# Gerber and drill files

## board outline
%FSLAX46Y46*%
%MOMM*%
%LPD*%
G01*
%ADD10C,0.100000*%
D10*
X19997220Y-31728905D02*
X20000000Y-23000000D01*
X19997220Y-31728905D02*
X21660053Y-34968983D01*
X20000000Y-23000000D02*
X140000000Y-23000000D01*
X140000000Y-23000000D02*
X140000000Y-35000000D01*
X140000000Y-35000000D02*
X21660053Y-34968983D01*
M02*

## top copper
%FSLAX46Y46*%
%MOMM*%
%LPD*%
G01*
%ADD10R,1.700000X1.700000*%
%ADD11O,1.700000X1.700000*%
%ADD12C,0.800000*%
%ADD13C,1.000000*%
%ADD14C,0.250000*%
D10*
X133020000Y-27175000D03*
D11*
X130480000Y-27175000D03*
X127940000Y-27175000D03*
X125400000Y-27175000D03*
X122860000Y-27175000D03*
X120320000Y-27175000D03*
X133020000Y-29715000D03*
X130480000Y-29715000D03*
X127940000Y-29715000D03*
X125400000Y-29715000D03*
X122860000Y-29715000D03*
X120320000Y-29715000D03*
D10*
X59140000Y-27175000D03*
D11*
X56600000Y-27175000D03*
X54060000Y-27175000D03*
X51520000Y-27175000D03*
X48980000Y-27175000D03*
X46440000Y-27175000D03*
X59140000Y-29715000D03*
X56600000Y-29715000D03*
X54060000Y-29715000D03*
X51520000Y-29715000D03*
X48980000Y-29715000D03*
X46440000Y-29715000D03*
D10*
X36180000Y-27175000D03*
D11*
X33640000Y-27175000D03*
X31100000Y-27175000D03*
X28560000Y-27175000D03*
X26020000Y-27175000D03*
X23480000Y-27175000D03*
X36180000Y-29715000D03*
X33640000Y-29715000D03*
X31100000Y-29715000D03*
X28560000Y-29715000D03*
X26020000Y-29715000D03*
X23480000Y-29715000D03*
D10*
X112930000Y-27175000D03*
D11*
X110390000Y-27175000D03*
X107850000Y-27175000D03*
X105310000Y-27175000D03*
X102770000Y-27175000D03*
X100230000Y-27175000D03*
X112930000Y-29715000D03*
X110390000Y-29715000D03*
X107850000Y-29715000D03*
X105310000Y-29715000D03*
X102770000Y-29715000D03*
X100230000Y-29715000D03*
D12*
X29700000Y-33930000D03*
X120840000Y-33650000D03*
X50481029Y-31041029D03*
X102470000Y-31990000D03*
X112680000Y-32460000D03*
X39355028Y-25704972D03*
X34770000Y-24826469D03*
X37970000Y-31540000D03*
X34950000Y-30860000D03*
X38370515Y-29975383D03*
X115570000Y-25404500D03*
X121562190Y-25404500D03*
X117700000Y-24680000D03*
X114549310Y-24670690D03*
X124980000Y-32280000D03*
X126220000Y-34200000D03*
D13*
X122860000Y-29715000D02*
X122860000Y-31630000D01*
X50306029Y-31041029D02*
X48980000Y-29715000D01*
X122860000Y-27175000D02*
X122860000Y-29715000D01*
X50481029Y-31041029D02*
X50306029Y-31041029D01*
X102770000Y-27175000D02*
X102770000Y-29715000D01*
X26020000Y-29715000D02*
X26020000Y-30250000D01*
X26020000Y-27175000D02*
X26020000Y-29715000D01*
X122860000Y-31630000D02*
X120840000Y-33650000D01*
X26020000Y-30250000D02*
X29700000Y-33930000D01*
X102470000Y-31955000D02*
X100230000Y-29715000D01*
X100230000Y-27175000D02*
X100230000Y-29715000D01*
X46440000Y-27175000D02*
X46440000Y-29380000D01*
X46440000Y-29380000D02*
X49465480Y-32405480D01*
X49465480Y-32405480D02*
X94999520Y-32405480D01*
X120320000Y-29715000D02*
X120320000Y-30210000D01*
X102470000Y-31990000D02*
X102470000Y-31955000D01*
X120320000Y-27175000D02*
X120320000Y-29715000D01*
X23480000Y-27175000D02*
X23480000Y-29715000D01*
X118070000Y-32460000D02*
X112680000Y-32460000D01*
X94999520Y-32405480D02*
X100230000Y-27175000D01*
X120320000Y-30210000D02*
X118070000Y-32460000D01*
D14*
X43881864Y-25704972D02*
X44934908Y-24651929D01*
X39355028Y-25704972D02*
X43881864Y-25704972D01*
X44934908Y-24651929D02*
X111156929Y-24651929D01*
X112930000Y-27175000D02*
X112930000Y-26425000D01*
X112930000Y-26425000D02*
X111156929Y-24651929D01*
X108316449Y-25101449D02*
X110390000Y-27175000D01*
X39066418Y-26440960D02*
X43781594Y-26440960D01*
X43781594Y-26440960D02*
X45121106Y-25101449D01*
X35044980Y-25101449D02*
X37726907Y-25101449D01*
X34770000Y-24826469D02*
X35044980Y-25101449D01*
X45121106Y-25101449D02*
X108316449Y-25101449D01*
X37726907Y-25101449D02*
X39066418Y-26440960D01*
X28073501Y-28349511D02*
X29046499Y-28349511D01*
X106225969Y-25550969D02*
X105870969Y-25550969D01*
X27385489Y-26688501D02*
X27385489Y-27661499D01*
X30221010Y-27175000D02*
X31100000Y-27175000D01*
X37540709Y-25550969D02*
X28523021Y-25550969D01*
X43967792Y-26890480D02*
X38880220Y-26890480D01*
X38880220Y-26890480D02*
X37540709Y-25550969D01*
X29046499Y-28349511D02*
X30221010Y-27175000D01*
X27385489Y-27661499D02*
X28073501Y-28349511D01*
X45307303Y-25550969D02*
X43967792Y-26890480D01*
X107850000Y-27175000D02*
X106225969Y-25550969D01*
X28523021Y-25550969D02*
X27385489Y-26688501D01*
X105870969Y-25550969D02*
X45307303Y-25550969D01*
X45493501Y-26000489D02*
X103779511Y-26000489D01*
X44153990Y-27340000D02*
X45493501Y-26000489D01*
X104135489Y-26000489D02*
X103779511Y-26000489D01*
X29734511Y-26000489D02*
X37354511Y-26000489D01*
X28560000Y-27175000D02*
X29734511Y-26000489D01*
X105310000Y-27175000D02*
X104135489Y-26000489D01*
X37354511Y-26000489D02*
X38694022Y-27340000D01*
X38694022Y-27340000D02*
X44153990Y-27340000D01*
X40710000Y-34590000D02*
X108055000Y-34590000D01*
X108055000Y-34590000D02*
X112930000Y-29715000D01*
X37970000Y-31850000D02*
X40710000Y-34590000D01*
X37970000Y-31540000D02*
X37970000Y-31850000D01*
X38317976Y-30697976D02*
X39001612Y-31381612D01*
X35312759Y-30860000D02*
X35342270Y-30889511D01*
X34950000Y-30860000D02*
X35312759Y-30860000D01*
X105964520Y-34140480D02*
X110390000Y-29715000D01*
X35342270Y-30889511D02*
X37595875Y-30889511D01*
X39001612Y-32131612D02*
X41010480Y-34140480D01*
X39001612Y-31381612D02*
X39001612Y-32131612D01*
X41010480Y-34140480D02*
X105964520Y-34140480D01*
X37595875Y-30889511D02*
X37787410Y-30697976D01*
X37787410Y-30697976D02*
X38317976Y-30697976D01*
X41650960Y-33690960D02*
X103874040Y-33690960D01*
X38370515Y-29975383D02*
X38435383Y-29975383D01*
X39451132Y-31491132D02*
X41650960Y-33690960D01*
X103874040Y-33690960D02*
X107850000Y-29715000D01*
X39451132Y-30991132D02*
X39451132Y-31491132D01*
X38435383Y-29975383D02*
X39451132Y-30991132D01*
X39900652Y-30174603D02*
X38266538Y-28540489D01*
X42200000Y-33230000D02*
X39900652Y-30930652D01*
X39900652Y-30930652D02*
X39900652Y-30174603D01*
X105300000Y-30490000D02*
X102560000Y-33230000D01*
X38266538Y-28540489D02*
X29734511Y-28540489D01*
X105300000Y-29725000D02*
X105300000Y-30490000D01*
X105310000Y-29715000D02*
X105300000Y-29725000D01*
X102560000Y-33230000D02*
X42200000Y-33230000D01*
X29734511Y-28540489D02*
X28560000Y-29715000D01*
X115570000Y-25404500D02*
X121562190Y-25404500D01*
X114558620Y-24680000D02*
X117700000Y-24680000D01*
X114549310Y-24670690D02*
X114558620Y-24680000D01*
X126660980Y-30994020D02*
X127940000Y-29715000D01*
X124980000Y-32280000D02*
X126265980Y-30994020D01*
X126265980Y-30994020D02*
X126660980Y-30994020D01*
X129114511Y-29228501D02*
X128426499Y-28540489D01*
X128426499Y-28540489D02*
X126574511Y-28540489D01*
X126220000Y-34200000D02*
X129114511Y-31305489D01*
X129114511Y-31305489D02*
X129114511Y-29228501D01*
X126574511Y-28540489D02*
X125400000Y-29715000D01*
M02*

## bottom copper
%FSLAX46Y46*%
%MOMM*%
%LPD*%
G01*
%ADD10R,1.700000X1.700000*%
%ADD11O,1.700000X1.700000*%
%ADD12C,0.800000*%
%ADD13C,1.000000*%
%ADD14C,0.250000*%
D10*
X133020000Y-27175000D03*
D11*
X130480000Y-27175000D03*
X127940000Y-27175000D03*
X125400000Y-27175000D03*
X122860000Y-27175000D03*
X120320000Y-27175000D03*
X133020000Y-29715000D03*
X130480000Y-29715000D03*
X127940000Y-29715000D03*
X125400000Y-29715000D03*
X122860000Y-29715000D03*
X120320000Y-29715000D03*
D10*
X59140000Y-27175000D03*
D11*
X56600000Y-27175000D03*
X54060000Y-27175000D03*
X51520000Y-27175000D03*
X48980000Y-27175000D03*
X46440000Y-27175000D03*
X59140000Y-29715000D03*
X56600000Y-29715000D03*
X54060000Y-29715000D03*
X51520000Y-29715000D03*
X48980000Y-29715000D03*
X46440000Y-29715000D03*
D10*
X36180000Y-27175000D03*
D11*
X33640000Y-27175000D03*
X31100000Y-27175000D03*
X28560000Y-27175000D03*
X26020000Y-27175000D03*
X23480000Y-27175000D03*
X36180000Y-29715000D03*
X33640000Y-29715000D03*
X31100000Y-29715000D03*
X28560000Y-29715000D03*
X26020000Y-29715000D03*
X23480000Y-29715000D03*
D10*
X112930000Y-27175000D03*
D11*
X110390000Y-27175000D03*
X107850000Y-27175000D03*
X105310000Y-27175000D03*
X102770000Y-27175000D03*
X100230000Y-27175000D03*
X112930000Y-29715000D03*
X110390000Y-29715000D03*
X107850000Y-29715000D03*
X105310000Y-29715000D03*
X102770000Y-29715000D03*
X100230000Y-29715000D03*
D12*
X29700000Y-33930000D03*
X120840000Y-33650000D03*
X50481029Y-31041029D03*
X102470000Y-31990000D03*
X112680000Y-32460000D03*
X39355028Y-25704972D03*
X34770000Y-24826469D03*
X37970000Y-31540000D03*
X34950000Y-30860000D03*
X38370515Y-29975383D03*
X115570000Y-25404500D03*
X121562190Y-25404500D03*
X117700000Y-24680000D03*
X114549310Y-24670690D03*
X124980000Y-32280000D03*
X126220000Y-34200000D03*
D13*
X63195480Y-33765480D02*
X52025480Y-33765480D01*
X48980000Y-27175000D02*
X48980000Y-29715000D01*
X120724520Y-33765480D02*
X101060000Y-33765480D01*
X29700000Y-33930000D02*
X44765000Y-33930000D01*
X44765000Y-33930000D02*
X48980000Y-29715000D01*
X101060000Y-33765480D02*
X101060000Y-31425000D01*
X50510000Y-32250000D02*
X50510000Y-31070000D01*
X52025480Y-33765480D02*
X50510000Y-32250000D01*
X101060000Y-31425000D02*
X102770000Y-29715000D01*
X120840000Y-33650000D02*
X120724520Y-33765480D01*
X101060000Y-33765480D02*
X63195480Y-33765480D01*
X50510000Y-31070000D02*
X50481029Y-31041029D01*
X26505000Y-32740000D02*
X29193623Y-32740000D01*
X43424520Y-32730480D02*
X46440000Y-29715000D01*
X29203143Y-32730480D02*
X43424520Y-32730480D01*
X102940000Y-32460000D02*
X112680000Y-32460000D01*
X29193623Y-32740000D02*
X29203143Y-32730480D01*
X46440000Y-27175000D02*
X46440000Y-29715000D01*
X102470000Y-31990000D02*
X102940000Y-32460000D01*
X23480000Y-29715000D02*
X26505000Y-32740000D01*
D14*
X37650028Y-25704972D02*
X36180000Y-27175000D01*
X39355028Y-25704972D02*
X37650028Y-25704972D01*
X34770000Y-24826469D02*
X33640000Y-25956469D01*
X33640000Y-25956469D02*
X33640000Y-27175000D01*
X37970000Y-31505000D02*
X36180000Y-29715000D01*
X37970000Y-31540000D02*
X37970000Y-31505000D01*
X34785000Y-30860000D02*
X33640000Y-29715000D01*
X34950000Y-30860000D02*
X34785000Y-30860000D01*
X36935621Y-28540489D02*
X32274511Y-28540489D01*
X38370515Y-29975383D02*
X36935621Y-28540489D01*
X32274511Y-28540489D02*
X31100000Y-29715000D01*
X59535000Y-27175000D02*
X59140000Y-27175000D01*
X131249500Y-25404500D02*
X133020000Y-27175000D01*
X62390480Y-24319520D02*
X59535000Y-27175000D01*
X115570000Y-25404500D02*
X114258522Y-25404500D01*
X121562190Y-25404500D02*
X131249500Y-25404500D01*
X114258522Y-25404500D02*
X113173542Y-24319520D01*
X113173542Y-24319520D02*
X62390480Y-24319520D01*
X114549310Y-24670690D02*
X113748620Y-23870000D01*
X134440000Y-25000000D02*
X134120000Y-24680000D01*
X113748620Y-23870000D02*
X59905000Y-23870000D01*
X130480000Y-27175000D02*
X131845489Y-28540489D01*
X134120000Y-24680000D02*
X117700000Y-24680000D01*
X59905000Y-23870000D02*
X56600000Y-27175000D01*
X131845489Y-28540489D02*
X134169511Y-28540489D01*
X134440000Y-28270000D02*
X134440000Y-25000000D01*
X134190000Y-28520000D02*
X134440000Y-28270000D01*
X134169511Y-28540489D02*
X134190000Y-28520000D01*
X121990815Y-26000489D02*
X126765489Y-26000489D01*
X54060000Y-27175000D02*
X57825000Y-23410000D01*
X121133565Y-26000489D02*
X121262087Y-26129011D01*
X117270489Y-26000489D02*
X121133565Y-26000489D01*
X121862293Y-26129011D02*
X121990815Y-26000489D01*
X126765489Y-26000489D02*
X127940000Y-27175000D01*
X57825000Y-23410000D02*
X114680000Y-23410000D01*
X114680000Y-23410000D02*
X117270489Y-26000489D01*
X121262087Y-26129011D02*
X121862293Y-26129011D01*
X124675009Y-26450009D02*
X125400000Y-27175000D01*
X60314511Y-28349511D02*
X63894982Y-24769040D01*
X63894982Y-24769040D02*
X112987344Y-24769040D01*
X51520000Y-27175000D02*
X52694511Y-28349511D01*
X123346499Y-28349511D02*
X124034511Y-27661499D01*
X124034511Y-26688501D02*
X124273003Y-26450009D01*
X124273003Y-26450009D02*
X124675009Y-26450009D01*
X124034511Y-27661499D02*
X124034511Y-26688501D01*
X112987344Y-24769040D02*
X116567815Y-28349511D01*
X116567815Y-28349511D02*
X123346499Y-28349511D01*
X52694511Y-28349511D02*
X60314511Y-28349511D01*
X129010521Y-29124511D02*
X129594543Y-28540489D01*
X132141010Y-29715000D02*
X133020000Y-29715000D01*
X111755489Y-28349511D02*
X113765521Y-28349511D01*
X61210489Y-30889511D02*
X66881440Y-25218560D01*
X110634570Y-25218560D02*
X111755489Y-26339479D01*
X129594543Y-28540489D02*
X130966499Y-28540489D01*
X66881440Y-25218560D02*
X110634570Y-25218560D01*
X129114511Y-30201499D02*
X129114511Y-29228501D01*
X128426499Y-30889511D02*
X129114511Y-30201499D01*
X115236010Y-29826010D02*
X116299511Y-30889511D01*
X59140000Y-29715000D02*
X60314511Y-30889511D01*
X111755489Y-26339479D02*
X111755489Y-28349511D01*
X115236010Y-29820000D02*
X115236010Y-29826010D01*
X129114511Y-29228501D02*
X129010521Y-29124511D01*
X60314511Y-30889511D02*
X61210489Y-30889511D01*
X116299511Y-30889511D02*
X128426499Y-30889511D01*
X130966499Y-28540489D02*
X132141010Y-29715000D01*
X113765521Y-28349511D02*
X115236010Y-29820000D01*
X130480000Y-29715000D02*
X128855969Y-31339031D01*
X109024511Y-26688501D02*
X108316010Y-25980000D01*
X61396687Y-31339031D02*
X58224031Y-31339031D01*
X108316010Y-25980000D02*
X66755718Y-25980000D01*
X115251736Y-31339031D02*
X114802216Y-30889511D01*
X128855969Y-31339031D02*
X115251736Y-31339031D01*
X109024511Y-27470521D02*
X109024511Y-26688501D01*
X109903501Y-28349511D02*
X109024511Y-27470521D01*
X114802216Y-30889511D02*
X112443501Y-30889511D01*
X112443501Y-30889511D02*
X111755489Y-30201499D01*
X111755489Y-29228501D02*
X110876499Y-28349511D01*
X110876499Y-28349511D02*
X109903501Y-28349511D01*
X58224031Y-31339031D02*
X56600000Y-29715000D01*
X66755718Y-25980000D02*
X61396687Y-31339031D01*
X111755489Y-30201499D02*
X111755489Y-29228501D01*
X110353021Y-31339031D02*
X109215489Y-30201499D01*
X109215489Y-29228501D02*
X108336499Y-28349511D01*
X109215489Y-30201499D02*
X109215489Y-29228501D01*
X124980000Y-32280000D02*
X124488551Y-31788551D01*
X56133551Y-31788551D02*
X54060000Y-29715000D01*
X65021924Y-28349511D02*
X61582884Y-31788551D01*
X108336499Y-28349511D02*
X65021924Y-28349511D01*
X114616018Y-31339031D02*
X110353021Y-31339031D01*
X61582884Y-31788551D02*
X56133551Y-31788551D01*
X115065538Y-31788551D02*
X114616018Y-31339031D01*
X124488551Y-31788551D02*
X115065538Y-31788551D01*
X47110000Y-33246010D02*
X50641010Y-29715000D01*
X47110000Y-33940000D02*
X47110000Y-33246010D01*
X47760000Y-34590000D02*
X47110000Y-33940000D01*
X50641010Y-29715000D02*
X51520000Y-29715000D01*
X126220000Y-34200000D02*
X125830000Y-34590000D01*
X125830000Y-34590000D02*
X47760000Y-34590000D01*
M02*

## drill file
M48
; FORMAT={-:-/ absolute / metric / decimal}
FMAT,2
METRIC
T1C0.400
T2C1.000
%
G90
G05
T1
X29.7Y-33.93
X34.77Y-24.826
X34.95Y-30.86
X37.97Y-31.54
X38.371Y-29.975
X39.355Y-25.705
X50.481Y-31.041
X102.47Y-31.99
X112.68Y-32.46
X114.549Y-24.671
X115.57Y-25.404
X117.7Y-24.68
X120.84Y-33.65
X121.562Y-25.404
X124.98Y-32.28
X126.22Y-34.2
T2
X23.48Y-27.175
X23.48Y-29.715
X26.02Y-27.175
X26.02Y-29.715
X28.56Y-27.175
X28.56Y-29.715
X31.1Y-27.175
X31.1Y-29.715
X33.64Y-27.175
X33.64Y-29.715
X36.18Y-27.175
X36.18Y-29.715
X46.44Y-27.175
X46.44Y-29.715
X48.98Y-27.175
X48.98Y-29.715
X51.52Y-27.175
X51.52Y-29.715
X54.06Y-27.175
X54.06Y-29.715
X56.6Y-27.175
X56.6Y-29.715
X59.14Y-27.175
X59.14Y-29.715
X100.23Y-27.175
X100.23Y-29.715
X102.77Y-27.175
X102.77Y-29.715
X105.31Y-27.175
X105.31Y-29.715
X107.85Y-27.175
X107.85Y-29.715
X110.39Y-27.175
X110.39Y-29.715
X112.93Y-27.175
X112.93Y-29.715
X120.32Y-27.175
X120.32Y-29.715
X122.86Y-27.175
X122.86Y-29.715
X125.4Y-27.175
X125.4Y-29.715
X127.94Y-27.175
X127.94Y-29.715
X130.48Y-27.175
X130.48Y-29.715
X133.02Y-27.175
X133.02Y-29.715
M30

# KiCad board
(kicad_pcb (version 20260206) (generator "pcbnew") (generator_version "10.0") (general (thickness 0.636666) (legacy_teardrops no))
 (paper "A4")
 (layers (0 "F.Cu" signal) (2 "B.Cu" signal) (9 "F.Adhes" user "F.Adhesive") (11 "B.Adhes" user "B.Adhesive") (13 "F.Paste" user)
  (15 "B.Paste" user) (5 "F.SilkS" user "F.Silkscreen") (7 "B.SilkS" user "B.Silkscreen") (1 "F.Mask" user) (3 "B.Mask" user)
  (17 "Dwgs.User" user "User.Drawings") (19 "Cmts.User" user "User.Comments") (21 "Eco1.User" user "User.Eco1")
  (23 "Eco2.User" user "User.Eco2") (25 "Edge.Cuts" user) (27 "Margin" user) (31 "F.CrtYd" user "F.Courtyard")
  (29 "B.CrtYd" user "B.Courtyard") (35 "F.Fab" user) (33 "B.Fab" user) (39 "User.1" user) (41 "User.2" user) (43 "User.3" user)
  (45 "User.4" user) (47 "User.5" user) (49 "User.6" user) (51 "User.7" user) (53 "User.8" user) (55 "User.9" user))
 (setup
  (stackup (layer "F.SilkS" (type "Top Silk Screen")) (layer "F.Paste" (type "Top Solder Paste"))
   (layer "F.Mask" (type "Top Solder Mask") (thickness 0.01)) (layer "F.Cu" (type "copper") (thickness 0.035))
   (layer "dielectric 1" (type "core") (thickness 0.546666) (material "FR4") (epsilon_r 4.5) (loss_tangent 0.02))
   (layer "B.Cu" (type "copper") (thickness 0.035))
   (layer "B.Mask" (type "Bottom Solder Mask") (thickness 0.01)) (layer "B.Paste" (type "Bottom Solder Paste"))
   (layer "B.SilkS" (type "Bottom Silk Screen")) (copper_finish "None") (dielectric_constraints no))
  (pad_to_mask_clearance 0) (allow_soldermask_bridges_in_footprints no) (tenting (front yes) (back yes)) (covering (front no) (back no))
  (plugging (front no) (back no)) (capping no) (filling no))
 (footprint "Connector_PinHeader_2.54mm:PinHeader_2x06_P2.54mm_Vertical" (layer "F.Cu") (at 133.02 27.175 -90)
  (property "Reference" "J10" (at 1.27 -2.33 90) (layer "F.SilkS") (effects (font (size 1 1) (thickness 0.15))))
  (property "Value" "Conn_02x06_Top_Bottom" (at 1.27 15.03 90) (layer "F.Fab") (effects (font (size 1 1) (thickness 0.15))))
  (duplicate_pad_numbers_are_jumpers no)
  (pad "1" thru_hole rect (at 0 0 270) (size 1.7 1.7) (drill 1) (layers "*.Cu" "*.Mask") (remove_unused_layers no) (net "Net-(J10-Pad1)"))
  (pad "2" thru_hole oval (at 0 2.54 270) (size 1.7 1.7) (drill 1) (layers "*.Cu" "*.Mask") (remove_unused_layers no) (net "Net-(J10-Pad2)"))
  (pad "3" thru_hole oval (at 0 5.08 270) (size 1.7 1.7) (drill 1) (layers "*.Cu" "*.Mask") (remove_unused_layers no) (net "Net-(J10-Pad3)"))
  (pad "4" thru_hole oval (at 0 7.62 270) (size 1.7 1.7) (drill 1) (layers "*.Cu" "*.Mask") (remove_unused_layers no) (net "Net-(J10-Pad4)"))
  (pad "5" thru_hole oval (at 0 10.16 270) (size 1.7 1.7) (drill 1) (layers "*.Cu" "*.Mask") (remove_unused_layers no) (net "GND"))
  (pad "6" thru_hole oval (at 0 12.7 270) (size 1.7 1.7) (drill 1) (layers "*.Cu" "*.Mask") (remove_unused_layers no) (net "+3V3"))
  (pad "7" thru_hole oval (at 2.54 0 270) (size 1.7 1.7) (drill 1) (layers "*.Cu" "*.Mask") (remove_unused_layers no) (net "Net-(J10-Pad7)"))
  (pad "8" thru_hole oval (at 2.54 2.54 270) (size 1.7 1.7) (drill 1) (layers "*.Cu" "*.Mask") (remove_unused_layers no)
   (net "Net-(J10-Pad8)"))
  (pad "9" thru_hole oval (at 2.54 5.08 270) (size 1.7 1.7) (drill 1) (layers "*.Cu" "*.Mask") (remove_unused_layers no)
   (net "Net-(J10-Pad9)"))
  (pad "10" thru_hole oval (at 2.54 7.62 270) (size 1.7 1.7) (drill 1) (layers "*.Cu" "*.Mask") (remove_unused_layers no)
   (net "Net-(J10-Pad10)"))
  (pad "11" thru_hole oval (at 2.54 10.16 270) (size 1.7 1.7) (drill 1) (layers "*.Cu" "*.Mask") (remove_unused_layers no) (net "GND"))
  (pad "12" thru_hole oval (at 2.54 12.7 270) (size 1.7 1.7) (drill 1) (layers "*.Cu" "*.Mask") (remove_unused_layers no) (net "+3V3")))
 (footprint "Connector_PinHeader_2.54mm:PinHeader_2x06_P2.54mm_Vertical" (layer "F.Cu") (at 59.14 27.175 -90)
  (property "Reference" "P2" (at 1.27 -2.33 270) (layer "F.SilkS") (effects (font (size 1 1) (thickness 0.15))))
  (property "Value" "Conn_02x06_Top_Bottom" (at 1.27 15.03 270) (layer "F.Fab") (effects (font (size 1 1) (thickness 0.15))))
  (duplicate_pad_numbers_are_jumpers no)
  (pad "1" thru_hole rect (at 0 0 270) (size 1.7 1.7) (drill 1) (layers "*.Cu" "*.Mask") (remove_unused_layers no) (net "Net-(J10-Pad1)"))
  (pad "2" thru_hole oval (at 0 2.54 270) (size 1.7 1.7) (drill 1) (layers "*.Cu" "*.Mask") (remove_unused_layers no) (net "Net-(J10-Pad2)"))
  (pad "3" thru_hole oval (at 0 5.08 270) (size 1.7 1.7) (drill 1) (layers "*.Cu" "*.Mask") (remove_unused_layers no) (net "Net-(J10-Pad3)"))
  (pad "4" thru_hole oval (at 0 7.62 270) (size 1.7 1.7) (drill 1) (layers "*.Cu" "*.Mask") (remove_unused_layers no) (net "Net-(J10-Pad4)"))
  (pad "5" thru_hole oval (at 0 10.16 270) (size 1.7 1.7) (drill 1) (layers "*.Cu" "*.Mask") (remove_unused_layers no) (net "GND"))
  (pad "6" thru_hole oval (at 0 12.7 270) (size 1.7 1.7) (drill 1) (layers "*.Cu" "*.Mask") (remove_unused_layers no) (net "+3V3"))
  (pad "7" thru_hole oval (at 2.54 0 270) (size 1.7 1.7) (drill 1) (layers "*.Cu" "*.Mask") (remove_unused_layers no) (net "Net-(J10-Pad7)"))
  (pad "8" thru_hole oval (at 2.54 2.54 270) (size 1.7 1.7) (drill 1) (layers "*.Cu" "*.Mask") (remove_unused_layers no)
   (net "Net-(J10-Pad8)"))
  (pad "9" thru_hole oval (at 2.54 5.08 270) (size 1.7 1.7) (drill 1) (layers "*.Cu" "*.Mask") (remove_unused_layers no)
   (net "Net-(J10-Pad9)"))
  (pad "10" thru_hole oval (at 2.54 7.62 270) (size 1.7 1.7) (drill 1) (layers "*.Cu" "*.Mask") (remove_unused_layers no)
   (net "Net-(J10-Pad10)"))
  (pad "11" thru_hole oval (at 2.54 10.16 270) (size 1.7 1.7) (drill 1) (layers "*.Cu" "*.Mask") (remove_unused_layers no) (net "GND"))
  (pad "12" thru_hole oval (at 2.54 12.7 270) (size 1.7 1.7) (drill 1) (layers "*.Cu" "*.Mask") (remove_unused_layers no) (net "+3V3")))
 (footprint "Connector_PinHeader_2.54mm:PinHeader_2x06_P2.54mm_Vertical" (layer "F.Cu") (at 36.18 27.175 -90)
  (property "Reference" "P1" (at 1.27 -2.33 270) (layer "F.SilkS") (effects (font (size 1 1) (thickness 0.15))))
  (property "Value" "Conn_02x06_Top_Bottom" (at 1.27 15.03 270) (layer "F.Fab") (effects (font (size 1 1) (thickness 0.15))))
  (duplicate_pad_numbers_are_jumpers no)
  (pad "1" thru_hole rect (at 0 0 270) (size 1.7 1.7) (drill 1) (layers "*.Cu" "*.Mask") (remove_unused_layers no) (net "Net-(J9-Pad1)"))
  (pad "2" thru_hole oval (at 0 2.54 270) (size 1.7 1.7) (drill 1) (layers "*.Cu" "*.Mask") (remove_unused_layers no) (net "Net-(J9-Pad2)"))
  (pad "3" thru_hole oval (at 0 5.08 270) (size 1.7 1.7) (drill 1) (layers "*.Cu" "*.Mask") (remove_unused_layers no) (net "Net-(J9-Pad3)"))
  (pad "4" thru_hole oval (at 0 7.62 270) (size 1.7 1.7) (drill 1) (layers "*.Cu" "*.Mask") (remove_unused_layers no) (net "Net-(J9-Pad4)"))
  (pad "5" thru_hole oval (at 0 10.16 270) (size 1.7 1.7) (drill 1) (layers "*.Cu" "*.Mask") (remove_unused_layers no) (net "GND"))
  (pad "6" thru_hole oval (at 0 12.7 270) (size 1.7 1.7) (drill 1) (layers "*.Cu" "*.Mask") (remove_unused_layers no) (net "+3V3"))
  (pad "7" thru_hole oval (at 2.54 0 270) (size 1.7 1.7) (drill 1) (layers "*.Cu" "*.Mask") (remove_unused_layers no) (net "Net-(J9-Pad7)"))
  (pad "8" thru_hole oval (at 2.54 2.54 270) (size 1.7 1.7) (drill 1) (layers "*.Cu" "*.Mask") (remove_unused_layers no)
   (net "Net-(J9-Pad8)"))
  (pad "9" thru_hole oval (at 2.54 5.08 270) (size 1.7 1.7) (drill 1) (layers "*.Cu" "*.Mask") (remove_unused_layers no)
   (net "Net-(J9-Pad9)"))
  (pad "10" thru_hole oval (at 2.54 7.62 270) (size 1.7 1.7) (drill 1) (layers "*.Cu" "*.Mask") (remove_unused_layers no)
   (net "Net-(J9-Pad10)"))
  (pad "11" thru_hole oval (at 2.54 10.16 270) (size 1.7 1.7) (drill 1) (layers "*.Cu" "*.Mask") (remove_unused_layers no) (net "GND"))
  (pad "12" thru_hole oval (at 2.54 12.7 270) (size 1.7 1.7) (drill 1) (layers "*.Cu" "*.Mask") (remove_unused_layers no) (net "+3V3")))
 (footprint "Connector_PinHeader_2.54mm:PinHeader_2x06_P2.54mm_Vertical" (layer "F.Cu") (at 112.93 27.175 -90)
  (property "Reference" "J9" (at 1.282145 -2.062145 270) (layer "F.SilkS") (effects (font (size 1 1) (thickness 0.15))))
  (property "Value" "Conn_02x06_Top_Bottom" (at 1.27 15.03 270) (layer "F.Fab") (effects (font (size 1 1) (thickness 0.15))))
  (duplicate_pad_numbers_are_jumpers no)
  (pad "1" thru_hole rect (at 0 0 270) (size 1.7 1.7) (drill 1) (layers "*.Cu" "*.Mask") (remove_unused_layers no) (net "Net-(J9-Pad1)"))
  (pad "2" thru_hole oval (at 0 2.54 270) (size 1.7 1.7) (drill 1) (layers "*.Cu" "*.Mask") (remove_unused_layers no) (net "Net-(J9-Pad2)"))
  (pad "3" thru_hole oval (at 0 5.08 270) (size 1.7 1.7) (drill 1) (layers "*.Cu" "*.Mask") (remove_unused_layers no) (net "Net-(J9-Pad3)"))
  (pad "4" thru_hole oval (at 0 7.62 270) (size 1.7 1.7) (drill 1) (layers "*.Cu" "*.Mask") (remove_unused_layers no) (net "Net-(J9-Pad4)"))
  (pad "5" thru_hole oval (at 0 10.16 270) (size 1.7 1.7) (drill 1) (layers "*.Cu" "*.Mask") (remove_unused_layers no) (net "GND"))
  (pad "6" thru_hole oval (at 0 12.7 270) (size 1.7 1.7) (drill 1) (layers "*.Cu" "*.Mask") (remove_unused_layers no) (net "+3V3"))
  (pad "7" thru_hole oval (at 2.54 0 270) (size 1.7 1.7) (drill 1) (layers "*.Cu" "*.Mask") (remove_unused_layers no) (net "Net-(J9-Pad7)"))
  (pad "8" thru_hole oval (at 2.54 2.54 270) (size 1.7 1.7) (drill 1) (layers "*.Cu" "*.Mask") (remove_unused_layers no)
   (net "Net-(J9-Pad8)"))
  (pad "9" thru_hole oval (at 2.54 5.08 270) (size 1.7 1.7) (drill 1) (layers "*.Cu" "*.Mask") (remove_unused_layers no)
   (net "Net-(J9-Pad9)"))
  (pad "10" thru_hole oval (at 2.54 7.62 270) (size 1.7 1.7) (drill 1) (layers "*.Cu" "*.Mask") (remove_unused_layers no)
   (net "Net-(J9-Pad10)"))
  (pad "11" thru_hole oval (at 2.54 10.16 270) (size 1.7 1.7) (drill 1) (layers "*.Cu" "*.Mask") (remove_unused_layers no) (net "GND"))
  (pad "12" thru_hole oval (at 2.54 12.7 270) (size 1.7 1.7) (drill 1) (layers "*.Cu" "*.Mask") (remove_unused_layers no) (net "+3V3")))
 (gr_line (start 19.99722 31.728905) (end 20 23) (stroke (width 0.1) (type solid)) (layer "Edge.Cuts"))
 (gr_line (start 19.99722 31.728905) (end 21.660053 34.968983) (stroke (width 0.1) (type solid)) (layer "Edge.Cuts"))
 (gr_line (start 20 23) (end 140 23) (stroke (width 0.1) (type solid)) (layer "Edge.Cuts"))
 (gr_line (start 140 23) (end 140 35) (stroke (width 0.1) (type solid)) (layer "Edge.Cuts"))
 (gr_line (start 140 35) (end 21.660053 34.968983) (stroke (width 0.1) (type solid)) (layer "Edge.Cuts"))
 (segment (start 122.86 29.715) (end 122.86 31.63) (width 1) (layer "F.Cu") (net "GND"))
 (segment (start 50.306029 31.041029) (end 48.98 29.715) (width 1) (layer "F.Cu") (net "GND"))
 (segment (start 122.86 27.175) (end 122.86 29.715) (width 1) (layer "F.Cu") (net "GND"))
 (segment (start 50.481029 31.041029) (end 50.306029 31.041029) (width 1) (layer "F.Cu") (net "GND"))
 (segment (start 102.77 27.175) (end 102.77 29.715) (width 1) (layer "F.Cu") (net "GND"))
 (segment (start 26.02 29.715) (end 26.02 30.25) (width 1) (layer "F.Cu") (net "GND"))
 (segment (start 26.02 27.175) (end 26.02 29.715) (width 1) (layer "F.Cu") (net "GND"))
 (segment (start 122.86 31.63) (end 120.84 33.65) (width 1) (layer "F.Cu") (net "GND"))
 (segment (start 26.02 30.25) (end 29.7 33.93) (width 1) (layer "F.Cu") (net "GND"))
 (via (at 29.7 33.93) (size 0.8) (drill 0.4) (layers "F.Cu" "B.Cu") (capping no) (covering (front no) (back no))
  (plugging (front no) (back no)) (filling no) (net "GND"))
 (via (at 120.84 33.65) (size 0.8) (drill 0.4) (layers "F.Cu" "B.Cu") (capping no) (covering (front no) (back no))
  (plugging (front no) (back no)) (filling no) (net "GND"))
 (via (at 50.481029 31.041029) (size 0.8) (drill 0.4) (layers "F.Cu" "B.Cu") (capping no) (covering (front no) (back no))
  (plugging (front no) (back no)) (filling no) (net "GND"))
 (segment (start 63.19548 33.76548) (end 52.02548 33.76548) (width 1) (layer "B.Cu") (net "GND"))
 (segment (start 48.98 27.175) (end 48.98 29.715) (width 1) (layer "B.Cu") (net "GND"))
 (segment (start 120.72452 33.76548) (end 101.06 33.76548) (width 1) (layer "B.Cu") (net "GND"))
 (segment (start 29.7 33.93) (end 44.765 33.93) (width 1) (layer "B.Cu") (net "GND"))
 (segment (start 44.765 33.93) (end 48.98 29.715) (width 1) (layer "B.Cu") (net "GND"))
 (segment (start 101.06 33.76548) (end 101.06 31.425) (width 1) (layer "B.Cu") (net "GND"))
 (segment (start 50.51 32.25) (end 50.51 31.07) (width 1) (layer "B.Cu") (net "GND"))
 (segment (start 52.02548 33.76548) (end 50.51 32.25) (width 1) (layer "B.Cu") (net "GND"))
 (segment (start 101.06 31.425) (end 102.77 29.715) (width 1) (layer "B.Cu") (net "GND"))
 (segment (start 120.84 33.65) (end 120.72452 33.76548) (width 1) (layer "B.Cu") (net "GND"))
 (segment (start 101.06 33.76548) (end 63.19548 33.76548) (width 1) (layer "B.Cu") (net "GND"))
 (segment (start 50.51 31.07) (end 50.481029 31.041029) (width 1) (layer "B.Cu") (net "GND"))
 (segment (start 102.47 31.955) (end 100.23 29.715) (width 1) (layer "F.Cu") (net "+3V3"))
 (segment (start 100.23 27.175) (end 100.23 29.715) (width 1) (layer "F.Cu") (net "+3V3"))
 (segment (start 46.44 27.175) (end 46.44 29.38) (width 1) (layer "F.Cu") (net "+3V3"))
 (segment (start 46.44 29.38) (end 49.46548 32.40548) (width 1) (layer "F.Cu") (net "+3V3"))
 (segment (start 49.46548 32.40548) (end 94.99952 32.40548) (width 1) (layer "F.Cu") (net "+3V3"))
 (segment (start 120.32 29.715) (end 120.32 30.21) (width 1) (layer "F.Cu") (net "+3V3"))
 (segment (start 102.47 31.99) (end 102.47 31.955) (width 1) (layer "F.Cu") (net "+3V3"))
 (segment (start 120.32 27.175) (end 120.32 29.715) (width 1) (layer "F.Cu") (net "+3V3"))
 (segment (start 23.48 27.175) (end 23.48 29.715) (width 1) (layer "F.Cu") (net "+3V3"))
 (segment (start 118.07 32.46) (end 112.68 32.46) (width 1) (layer "F.Cu") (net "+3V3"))
 (segment (start 94.99952 32.40548) (end 100.23 27.175) (width 1) (layer "F.Cu") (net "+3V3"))
 (segment (start 120.32 30.21) (end 118.07 32.46) (width 1) (layer "F.Cu") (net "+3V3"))
 (via (at 102.47 31.99) (size 0.8) (drill 0.4) (layers "F.Cu" "B.Cu") (capping no) (covering (front no) (back no))
  (plugging (front no) (back no)) (filling no) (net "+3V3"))
 (via (at 112.68 32.46) (size 0.8) (drill 0.4) (layers "F.Cu" "B.Cu") (capping no) (covering (front no) (back no))
  (plugging (front no) (back no)) (filling no) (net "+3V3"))
 (segment (start 26.505 32.74) (end 29.193623 32.74) (width 1) (layer "B.Cu") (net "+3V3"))
 (segment (start 43.42452 32.73048) (end 46.44 29.715) (width 1) (layer "B.Cu") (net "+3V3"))
 (segment (start 29.203143 32.73048) (end 43.42452 32.73048) (width 1) (layer "B.Cu") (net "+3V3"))
 (segment (start 102.94 32.46) (end 112.68 32.46) (width 1) (layer "B.Cu") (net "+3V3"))
 (segment (start 29.193623 32.74) (end 29.203143 32.73048) (width 1) (layer "B.Cu") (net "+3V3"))
 (segment (start 46.44 27.175) (end 46.44 29.715) (width 1) (layer "B.Cu") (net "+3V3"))
 (segment (start 102.47 31.99) (end 102.94 32.46) (width 1) (layer "B.Cu") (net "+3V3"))
 (segment (start 23.48 29.715) (end 26.505 32.74) (width 1) (layer "B.Cu") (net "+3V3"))
 (segment (start 43.881864 25.704972) (end 44.934908 24.651929) (width 0.25) (layer "F.Cu") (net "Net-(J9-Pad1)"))
 (segment (start 39.355028 25.704972) (end 43.881864 25.704972) (width 0.25) (layer "F.Cu") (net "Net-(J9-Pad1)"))
 (segment (start 44.934908 24.651929) (end 111.156929 24.651929) (width 0.25) (layer "F.Cu") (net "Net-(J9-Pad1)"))
 (segment (start 112.93 27.175) (end 112.93 26.425) (width 0.25) (layer "F.Cu") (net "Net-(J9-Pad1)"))
 (segment (start 112.93 26.425) (end 111.156929 24.651929) (width 0.25) (layer "F.Cu") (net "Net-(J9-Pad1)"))
 (via (at 39.355028 25.704972) (size 0.8) (drill 0.4) (layers "F.Cu" "B.Cu") (capping no) (covering (front no) (back no))
  (plugging (front no) (back no)) (filling no) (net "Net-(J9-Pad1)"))
 (segment (start 37.650028 25.704972) (end 36.18 27.175) (width 0.25) (layer "B.Cu") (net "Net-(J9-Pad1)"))
 (segment (start 39.355028 25.704972) (end 37.650028 25.704972) (width 0.25) (layer "B.Cu") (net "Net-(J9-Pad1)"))
 (segment (start 108.316449 25.101449) (end 110.39 27.175) (width 0.25) (layer "F.Cu") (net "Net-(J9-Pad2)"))
 (segment (start 39.066418 26.44096) (end 43.781594 26.44096) (width 0.25) (layer "F.Cu") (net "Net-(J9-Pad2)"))
 (segment (start 43.781594 26.44096) (end 45.121106 25.101449) (width 0.25) (layer "F.Cu") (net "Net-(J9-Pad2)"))
 (segment (start 35.04498 25.101449) (end 37.726907 25.101449) (width 0.25) (layer "F.Cu") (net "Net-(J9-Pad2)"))
 (segment (start 34.77 24.826469) (end 35.04498 25.101449) (width 0.25) (layer "F.Cu") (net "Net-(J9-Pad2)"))
 (segment (start 45.121106 25.101449) (end 108.316449 25.101449) (width 0.25) (layer "F.Cu") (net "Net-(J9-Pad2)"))
 (segment (start 37.726907 25.101449) (end 39.066418 26.44096) (width 0.25) (layer "F.Cu") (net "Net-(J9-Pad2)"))
 (via (at 34.77 24.826469) (size 0.8) (drill 0.4) (layers "F.Cu" "B.Cu") (capping no) (covering (front no) (back no))
  (plugging (front no) (back no)) (filling no) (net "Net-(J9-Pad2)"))
 (segment (start 34.77 24.826469) (end 33.64 25.956469) (width 0.25) (layer "B.Cu") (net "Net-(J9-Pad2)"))
 (segment (start 33.64 25.956469) (end 33.64 27.175) (width 0.25) (layer "B.Cu") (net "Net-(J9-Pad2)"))
 (segment (start 28.073501 28.349511) (end 29.046499 28.349511) (width 0.25) (layer "F.Cu") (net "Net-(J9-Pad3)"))
 (segment (start 106.225969 25.550969) (end 105.870969 25.550969) (width 0.25) (layer "F.Cu") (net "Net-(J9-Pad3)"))
 (segment (start 27.385489 26.688501) (end 27.385489 27.661499) (width 0.25) (layer "F.Cu") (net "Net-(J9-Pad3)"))
 (segment (start 30.22101 27.175) (end 31.1 27.175) (width 0.25) (layer "F.Cu") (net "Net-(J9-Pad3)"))
 (segment (start 37.540709 25.550969) (end 28.523021 25.550969) (width 0.25) (layer "F.Cu") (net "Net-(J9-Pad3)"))
 (segment (start 43.967792 26.89048) (end 38.88022 26.89048) (width 0.25) (layer "F.Cu") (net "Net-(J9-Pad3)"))
 (segment (start 38.88022 26.89048) (end 37.540709 25.550969) (width 0.25) (layer "F.Cu") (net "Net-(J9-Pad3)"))
 (segment (start 29.046499 28.349511) (end 30.22101 27.175) (width 0.25) (layer "F.Cu") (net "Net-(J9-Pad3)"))
 (segment (start 27.385489 27.661499) (end 28.073501 28.349511) (width 0.25) (layer "F.Cu") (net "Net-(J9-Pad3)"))
 (segment (start 45.307303 25.550969) (end 43.967792 26.89048) (width 0.25) (layer "F.Cu") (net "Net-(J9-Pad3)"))
 (segment (start 107.85 27.175) (end 106.225969 25.550969) (width 0.25) (layer "F.Cu") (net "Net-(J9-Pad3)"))
 (segment (start 28.523021 25.550969) (end 27.385489 26.688501) (width 0.25) (layer "F.Cu") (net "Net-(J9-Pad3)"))
 (segment (start 105.870969 25.550969) (end 45.307303 25.550969) (width 0.25) (layer "F.Cu") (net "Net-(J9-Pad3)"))
 (segment (start 45.493501 26.000489) (end 103.779511 26.000489) (width 0.25) (layer "F.Cu") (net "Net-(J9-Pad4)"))
 (segment (start 44.15399 27.34) (end 45.493501 26.000489) (width 0.25) (layer "F.Cu") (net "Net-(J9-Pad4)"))
 (segment (start 104.135489 26.000489) (end 103.779511 26.000489) (width 0.25) (layer "F.Cu") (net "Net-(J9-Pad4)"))
 (segment (start 29.734511 26.000489) (end 37.354511 26.000489) (width 0.25) (layer "F.Cu") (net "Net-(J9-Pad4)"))
 (segment (start 28.56 27.175) (end 29.734511 26.000489) (width 0.25) (layer "F.Cu") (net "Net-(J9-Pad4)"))
 (segment (start 105.31 27.175) (end 104.135489 26.000489) (width 0.25) (layer "F.Cu") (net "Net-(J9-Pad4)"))
 (segment (start 37.354511 26.000489) (end 38.694022 27.34) (width 0.25) (layer "F.Cu") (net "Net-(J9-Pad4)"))
 (segment (start 38.694022 27.34) (end 44.15399 27.34) (width 0.25) (layer "F.Cu") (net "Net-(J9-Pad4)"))
 (segment (start 40.71 34.59) (end 108.055 34.59) (width 0.25) (layer "F.Cu") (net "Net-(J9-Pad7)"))
 (segment (start 108.055 34.59) (end 112.93 29.715) (width 0.25) (layer "F.Cu") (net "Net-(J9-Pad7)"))
 (segment (start 37.97 31.85) (end 40.71 34.59) (width 0.25) (layer "F.Cu") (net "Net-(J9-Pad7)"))
 (segment (start 37.97 31.54) (end 37.97 31.85) (width 0.25) (layer "F.Cu") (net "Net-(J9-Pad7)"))
 (via (at 37.97 31.54) (size 0.8) (drill 0.4) (layers "F.Cu" "B.Cu") (capping no) (covering (front no) (back no))
  (plugging (front no) (back no)) (filling no) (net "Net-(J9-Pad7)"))
 (segment (start 37.97 31.505) (end 36.18 29.715) (width 0.25) (layer "B.Cu") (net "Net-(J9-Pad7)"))
 (segment (start 37.97 31.54) (end 37.97 31.505) (width 0.25) (layer "B.Cu") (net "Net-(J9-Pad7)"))
 (segment (start 38.317976 30.697976) (end 39.001612 31.381612) (width 0.25) (layer "F.Cu") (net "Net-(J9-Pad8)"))
 (segment (start 35.312759 30.86) (end 35.34227 30.889511) (width 0.25) (layer "F.Cu") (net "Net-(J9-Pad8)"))
 (segment (start 34.95 30.86) (end 35.312759 30.86) (width 0.25) (layer "F.Cu") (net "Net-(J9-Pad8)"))
 (segment (start 105.96452 34.14048) (end 110.39 29.715) (width 0.25) (layer "F.Cu") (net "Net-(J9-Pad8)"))
 (segment (start 35.34227 30.889511) (end 37.595875 30.889511) (width 0.25) (layer "F.Cu") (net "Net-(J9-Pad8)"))
 (segment (start 39.001612 32.131612) (end 41.01048 34.14048) (width 0.25) (layer "F.Cu") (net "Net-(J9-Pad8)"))
 (segment (start 39.001612 31.381612) (end 39.001612 32.131612) (width 0.25) (layer "F.Cu") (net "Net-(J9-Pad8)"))
 (segment (start 41.01048 34.14048) (end 105.96452 34.14048) (width 0.25) (layer "F.Cu") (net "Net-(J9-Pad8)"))
 (segment (start 37.595875 30.889511) (end 37.78741 30.697976) (width 0.25) (layer "F.Cu") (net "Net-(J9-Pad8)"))
 (segment (start 37.78741 30.697976) (end 38.317976 30.697976) (width 0.25) (layer "F.Cu") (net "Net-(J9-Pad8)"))
 (via (at 34.95 30.86) (size 0.8) (drill 0.4) (layers "F.Cu" "B.Cu") (capping no) (covering (front no) (back no))
  (plugging (front no) (back no)) (filling no) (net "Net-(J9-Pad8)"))
 (segment (start 34.785 30.86) (end 33.64 29.715) (width 0.25) (layer "B.Cu") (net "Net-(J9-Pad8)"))
 (segment (start 34.95 30.86) (end 34.785 30.86) (width 0.25) (layer "B.Cu") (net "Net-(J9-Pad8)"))
 (segment (start 41.65096 33.69096) (end 103.87404 33.69096) (width 0.25) (layer "F.Cu") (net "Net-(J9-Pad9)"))
 (segment (start 38.370515 29.975383) (end 38.435383 29.975383) (width 0.25) (layer "F.Cu") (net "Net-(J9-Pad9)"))
 (segment (start 39.451132 31.491132) (end 41.65096 33.69096) (width 0.25) (layer "F.Cu") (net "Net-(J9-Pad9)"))
 (segment (start 103.87404 33.69096) (end 107.85 29.715) (width 0.25) (layer "F.Cu") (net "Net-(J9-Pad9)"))
 (segment (start 39.451132 30.991132) (end 39.451132 31.491132) (width 0.25) (layer "F.Cu") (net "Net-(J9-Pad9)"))
 (segment (start 38.435383 29.975383) (end 39.451132 30.991132) (width 0.25) (layer "F.Cu") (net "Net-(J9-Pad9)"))
 (via (at 38.370515 29.975383) (size 0.8) (drill 0.4) (layers "F.Cu" "B.Cu") (capping no) (covering (front no) (back no))
  (plugging (front no) (back no)) (filling no) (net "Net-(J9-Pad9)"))
 (segment (start 36.935621 28.540489) (end 32.274511 28.540489) (width 0.25) (layer "B.Cu") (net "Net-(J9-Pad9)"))
 (segment (start 38.370515 29.975383) (end 36.935621 28.540489) (width 0.25) (layer "B.Cu") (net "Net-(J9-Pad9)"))
 (segment (start 32.274511 28.540489) (end 31.1 29.715) (width 0.25) (layer "B.Cu") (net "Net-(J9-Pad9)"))
 (segment (start 39.900652 30.174603) (end 38.266538 28.540489) (width 0.25) (layer "F.Cu") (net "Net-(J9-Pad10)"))
 (segment (start 42.2 33.23) (end 39.900652 30.930652) (width 0.25) (layer "F.Cu") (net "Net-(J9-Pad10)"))
 (segment (start 39.900652 30.930652) (end 39.900652 30.174603) (width 0.25) (layer "F.Cu") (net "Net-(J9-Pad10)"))
 (segment (start 105.3 30.49) (end 102.56 33.23) (width 0.25) (layer "F.Cu") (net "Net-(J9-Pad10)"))
 (segment (start 38.266538 28.540489) (end 29.734511 28.540489) (width 0.25) (layer "F.Cu") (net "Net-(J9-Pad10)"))
 (segment (start 105.3 29.725) (end 105.3 30.49) (width 0.25) (layer "F.Cu") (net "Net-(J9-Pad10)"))
 (segment (start 105.31 29.715) (end 105.3 29.725) (width 0.25) (layer "F.Cu") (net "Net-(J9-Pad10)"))
 (segment (start 102.56 33.23) (end 42.2 33.23) (width 0.25) (layer "F.Cu") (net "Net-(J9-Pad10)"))
 (segment (start 29.734511 28.540489) (end 28.56 29.715) (width 0.25) (layer "F.Cu") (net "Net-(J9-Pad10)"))
 (segment (start 115.57 25.4045) (end 121.56219 25.4045) (width 0.25) (layer "F.Cu") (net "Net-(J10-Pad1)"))
 (via (at 115.57 25.4045) (size 0.8) (drill 0.4) (layers "F.Cu" "B.Cu") (capping no) (covering (front no) (back no))
  (plugging (front no) (back no)) (filling no) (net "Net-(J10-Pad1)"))
 (via (at 121.56219 25.4045) (size 0.8) (drill 0.4) (layers "F.Cu" "B.Cu") (capping no) (covering (front no) (back no))
  (plugging (front no) (back no)) (filling no) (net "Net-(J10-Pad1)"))
 (segment (start 59.535 27.175) (end 59.14 27.175) (width 0.25) (layer "B.Cu") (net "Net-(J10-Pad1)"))
 (segment (start 131.2495 25.4045) (end 133.02 27.175) (width 0.25) (layer "B.Cu") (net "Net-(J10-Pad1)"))
 (segment (start 62.39048 24.31952) (end 59.535 27.175) (width 0.25) (layer "B.Cu") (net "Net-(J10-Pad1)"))
 (segment (start 115.57 25.4045) (end 114.258522 25.4045) (width 0.25) (layer "B.Cu") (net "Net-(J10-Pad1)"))
 (segment (start 121.56219 25.4045) (end 131.2495 25.4045) (width 0.25) (layer "B.Cu") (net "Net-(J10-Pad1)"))
 (segment (start 114.258522 25.4045) (end 113.173542 24.31952) (width 0.25) (layer "B.Cu") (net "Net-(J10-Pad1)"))
 (segment (start 113.173542 24.31952) (end 62.39048 24.31952) (width 0.25) (layer "B.Cu") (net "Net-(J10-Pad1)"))
 (segment (start 114.55862 24.68) (end 117.7 24.68) (width 0.25) (layer "F.Cu") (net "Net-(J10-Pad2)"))
 (segment (start 114.54931 24.67069) (end 114.55862 24.68) (width 0.25) (layer "F.Cu") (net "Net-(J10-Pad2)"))
 (via (at 117.7 24.68) (size 0.8) (drill 0.4) (layers "F.Cu" "B.Cu") (capping no) (covering (front no) (back no))
  (plugging (front no) (back no)) (filling no) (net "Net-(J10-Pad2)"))
 (via (at 114.54931 24.67069) (size 0.8) (drill 0.4) (layers "F.Cu" "B.Cu") (capping no) (covering (front no) (back no))
  (plugging (front no) (back no)) (filling no) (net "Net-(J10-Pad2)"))
 (segment (start 114.54931 24.67069) (end 113.74862 23.87) (width 0.25) (layer "B.Cu") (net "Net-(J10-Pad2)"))
 (segment (start 134.44 25) (end 134.12 24.68) (width 0.25) (layer "B.Cu") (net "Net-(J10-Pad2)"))
 (segment (start 113.74862 23.87) (end 59.905 23.87) (width 0.25) (layer "B.Cu") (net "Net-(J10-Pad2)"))
 (segment (start 130.48 27.175) (end 131.845489 28.540489) (width 0.25) (layer "B.Cu") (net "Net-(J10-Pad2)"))
 (segment (start 134.12 24.68) (end 117.7 24.68) (width 0.25) (layer "B.Cu") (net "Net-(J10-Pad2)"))
 (segment (start 59.905 23.87) (end 56.6 27.175) (width 0.25) (layer "B.Cu") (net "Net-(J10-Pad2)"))
 (segment (start 131.845489 28.540489) (end 134.169511 28.540489) (width 0.25) (layer "B.Cu") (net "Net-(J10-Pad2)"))
 (segment (start 134.44 28.27) (end 134.44 25) (width 0.25) (layer "B.Cu") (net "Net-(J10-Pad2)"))
 (segment (start 134.19 28.52) (end 134.44 28.27) (width 0.25) (layer "B.Cu") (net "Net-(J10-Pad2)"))
 (segment (start 134.169511 28.540489) (end 134.19 28.52) (width 0.25) (layer "B.Cu") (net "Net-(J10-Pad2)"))
 (segment (start 121.990815 26.000489) (end 126.765489 26.000489) (width 0.25) (layer "B.Cu") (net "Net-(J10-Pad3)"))
 (segment (start 54.06 27.175) (end 57.825 23.41) (width 0.25) (layer "B.Cu") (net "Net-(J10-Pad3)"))
 (segment (start 121.133565 26.000489) (end 121.262087 26.129011) (width 0.25) (layer "B.Cu") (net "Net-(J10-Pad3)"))
 (segment (start 117.270489 26.000489) (end 121.133565 26.000489) (width 0.25) (layer "B.Cu") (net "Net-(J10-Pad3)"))
 (segment (start 121.862293 26.129011) (end 121.990815 26.000489) (width 0.25) (layer "B.Cu") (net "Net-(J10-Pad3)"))
 (segment (start 126.765489 26.000489) (end 127.94 27.175) (width 0.25) (layer "B.Cu") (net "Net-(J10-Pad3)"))
 (segment (start 57.825 23.41) (end 114.68 23.41) (width 0.25) (layer "B.Cu") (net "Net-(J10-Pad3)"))
 (segment (start 114.68 23.41) (end 117.270489 26.000489) (width 0.25) (layer "B.Cu") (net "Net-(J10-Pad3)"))
 (segment (start 121.262087 26.129011) (end 121.862293 26.129011) (width 0.25) (layer "B.Cu") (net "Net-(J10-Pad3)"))
 (segment (start 124.675009 26.450009) (end 125.4 27.175) (width 0.25) (layer "B.Cu") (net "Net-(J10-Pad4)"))
 (segment (start 60.314511 28.349511) (end 63.894982 24.76904) (width 0.25) (layer "B.Cu") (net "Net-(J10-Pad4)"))
 (segment (start 63.894982 24.76904) (end 112.987344 24.76904) (width 0.25) (layer "B.Cu") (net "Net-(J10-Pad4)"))
 (segment (start 51.52 27.175) (end 52.694511 28.349511) (width 0.25) (layer "B.Cu") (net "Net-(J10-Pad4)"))
 (segment (start 123.346499 28.349511) (end 124.034511 27.661499) (width 0.25) (layer "B.Cu") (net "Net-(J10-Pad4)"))
 (segment (start 124.034511 26.688501) (end 124.273003 26.450009) (width 0.25) (layer "B.Cu") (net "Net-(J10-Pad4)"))
 (segment (start 124.273003 26.450009) (end 124.675009 26.450009) (width 0.25) (layer "B.Cu") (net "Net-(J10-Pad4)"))
 (segment (start 124.034511 27.661499) (end 124.034511 26.688501) (width 0.25) (layer "B.Cu") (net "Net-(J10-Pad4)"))
 (segment (start 112.987344 24.76904) (end 116.567815 28.349511) (width 0.25) (layer "B.Cu") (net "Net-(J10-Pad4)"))
 (segment (start 116.567815 28.349511) (end 123.346499 28.349511) (width 0.25) (layer "B.Cu") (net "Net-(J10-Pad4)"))
 (segment (start 52.694511 28.349511) (end 60.314511 28.349511) (width 0.25) (layer "B.Cu") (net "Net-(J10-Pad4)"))
 (segment (start 129.010521 29.124511) (end 129.594543 28.540489) (width 0.25) (layer "B.Cu") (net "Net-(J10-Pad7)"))
 (segment (start 132.14101 29.715) (end 133.02 29.715) (width 0.25) (layer "B.Cu") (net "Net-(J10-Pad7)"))
 (segment (start 111.755489 28.349511) (end 113.765521 28.349511) (width 0.25) (layer "B.Cu") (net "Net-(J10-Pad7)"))
 (segment (start 61.210489 30.889511) (end 66.88144 25.21856) (width 0.25) (layer "B.Cu") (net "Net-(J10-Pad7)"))
 (segment (start 110.63457 25.21856) (end 111.755489 26.339479) (width 0.25) (layer "B.Cu") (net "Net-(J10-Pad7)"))
 (segment (start 129.594543 28.540489) (end 130.966499 28.540489) (width 0.25) (layer "B.Cu") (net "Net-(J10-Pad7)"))
 (segment (start 66.88144 25.21856) (end 110.63457 25.21856) (width 0.25) (layer "B.Cu") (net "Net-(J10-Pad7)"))
 (segment (start 129.114511 30.201499) (end 129.114511 29.228501) (width 0.25) (layer "B.Cu") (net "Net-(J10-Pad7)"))
 (segment (start 128.426499 30.889511) (end 129.114511 30.201499) (width 0.25) (layer "B.Cu") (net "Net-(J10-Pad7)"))
 (segment (start 115.23601 29.82601) (end 116.299511 30.889511) (width 0.25) (layer "B.Cu") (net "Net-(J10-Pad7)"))
 (segment (start 59.14 29.715) (end 60.314511 30.889511) (width 0.25) (layer "B.Cu") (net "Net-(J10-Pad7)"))
 (segment (start 111.755489 26.339479) (end 111.755489 28.349511) (width 0.25) (layer "B.Cu") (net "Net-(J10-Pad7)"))
 (segment (start 115.23601 29.82) (end 115.23601 29.82601) (width 0.25) (layer "B.Cu") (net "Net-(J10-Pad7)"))
 (segment (start 129.114511 29.228501) (end 129.010521 29.124511) (width 0.25) (layer "B.Cu") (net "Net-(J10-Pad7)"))
 (segment (start 60.314511 30.889511) (end 61.210489 30.889511) (width 0.25) (layer "B.Cu") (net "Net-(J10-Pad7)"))
 (segment (start 116.299511 30.889511) (end 128.426499 30.889511) (width 0.25) (layer "B.Cu") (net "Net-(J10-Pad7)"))
 (segment (start 130.966499 28.540489) (end 132.14101 29.715) (width 0.25) (layer "B.Cu") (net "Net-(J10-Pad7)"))
 (segment (start 113.765521 28.349511) (end 115.23601 29.82) (width 0.25) (layer "B.Cu") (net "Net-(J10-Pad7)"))
 (segment (start 130.48 29.715) (end 128.855969 31.339031) (width 0.25) (layer "B.Cu") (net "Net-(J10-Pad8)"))
 (segment (start 109.024511 26.688501) (end 108.31601 25.98) (width 0.25) (layer "B.Cu") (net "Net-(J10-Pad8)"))
 (segment (start 61.396687 31.339031) (end 58.224031 31.339031) (width 0.25) (layer "B.Cu") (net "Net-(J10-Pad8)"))
 (segment (start 108.31601 25.98) (end 66.755718 25.98) (width 0.25) (layer "B.Cu") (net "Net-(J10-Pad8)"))
 (segment (start 115.251736 31.339031) (end 114.802216 30.889511) (width 0.25) (layer "B.Cu") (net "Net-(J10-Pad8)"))
 (segment (start 128.855969 31.339031) (end 115.251736 31.339031) (width 0.25) (layer "B.Cu") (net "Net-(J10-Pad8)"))
 (segment (start 109.024511 27.470521) (end 109.024511 26.688501) (width 0.25) (layer "B.Cu") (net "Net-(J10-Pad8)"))
 (segment (start 109.903501 28.349511) (end 109.024511 27.470521) (width 0.25) (layer "B.Cu") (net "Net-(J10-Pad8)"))
 (segment (start 114.802216 30.889511) (end 112.443501 30.889511) (width 0.25) (layer "B.Cu") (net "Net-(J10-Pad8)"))
 (segment (start 112.443501 30.889511) (end 111.755489 30.201499) (width 0.25) (layer "B.Cu") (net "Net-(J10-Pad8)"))
 (segment (start 111.755489 29.228501) (end 110.876499 28.349511) (width 0.25) (layer "B.Cu") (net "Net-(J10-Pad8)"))
 (segment (start 110.876499 28.349511) (end 109.903501 28.349511) (width 0.25) (layer "B.Cu") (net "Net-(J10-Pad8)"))
 (segment (start 58.224031 31.339031) (end 56.6 29.715) (width 0.25) (layer "B.Cu") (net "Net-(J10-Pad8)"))
 (segment (start 66.755718 25.98) (end 61.396687 31.339031) (width 0.25) (layer "B.Cu") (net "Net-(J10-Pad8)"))
 (segment (start 111.755489 30.201499) (end 111.755489 29.228501) (width 0.25) (layer "B.Cu") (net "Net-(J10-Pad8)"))
 (segment (start 126.66098 30.99402) (end 127.94 29.715) (width 0.25) (layer "F.Cu") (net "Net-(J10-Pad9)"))
 (segment (start 124.98 32.28) (end 126.26598 30.99402) (width 0.25) (layer "F.Cu") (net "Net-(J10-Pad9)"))
 (segment (start 126.26598 30.99402) (end 126.66098 30.99402) (width 0.25) (layer "F.Cu") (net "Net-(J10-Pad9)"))
 (via (at 124.98 32.28) (size 0.8) (drill 0.4) (layers "F.Cu" "B.Cu") (capping no) (covering (front no) (back no))
  (plugging (front no) (back no)) (filling no) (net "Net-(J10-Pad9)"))
 (segment (start 110.353021 31.339031) (end 109.215489 30.201499) (width 0.25) (layer "B.Cu") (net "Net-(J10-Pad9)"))
 (segment (start 109.215489 29.228501) (end 108.336499 28.349511) (width 0.25) (layer "B.Cu") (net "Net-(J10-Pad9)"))
 (segment (start 109.215489 30.201499) (end 109.215489 29.228501) (width 0.25) (layer "B.Cu") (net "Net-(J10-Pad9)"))
 (segment (start 124.98 32.28) (end 124.488551 31.788551) (width 0.25) (layer "B.Cu") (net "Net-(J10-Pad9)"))
 (segment (start 56.133551 31.788551) (end 54.06 29.715) (width 0.25) (layer "B.Cu") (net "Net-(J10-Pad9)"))
 (segment (start 65.021924 28.349511) (end 61.582884 31.788551) (width 0.25) (layer "B.Cu") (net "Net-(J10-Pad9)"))
 (segment (start 108.336499 28.349511) (end 65.021924 28.349511) (width 0.25) (layer "B.Cu") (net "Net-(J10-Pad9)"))
 (segment (start 114.616018 31.339031) (end 110.353021 31.339031) (width 0.25) (layer "B.Cu") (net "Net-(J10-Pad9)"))
 (segment (start 61.582884 31.788551) (end 56.133551 31.788551) (width 0.25) (layer "B.Cu") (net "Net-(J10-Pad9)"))
 (segment (start 115.065538 31.788551) (end 114.616018 31.339031) (width 0.25) (layer "B.Cu") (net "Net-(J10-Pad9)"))
 (segment (start 124.488551 31.788551) (end 115.065538 31.788551) (width 0.25) (layer "B.Cu") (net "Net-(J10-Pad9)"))
 (segment (start 129.114511 29.228501) (end 128.426499 28.540489) (width 0.25) (layer "F.Cu") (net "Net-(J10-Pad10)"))
 (segment (start 128.426499 28.540489) (end 126.574511 28.540489) (width 0.25) (layer "F.Cu") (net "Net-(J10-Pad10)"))
 (segment (start 126.22 34.2) (end 129.114511 31.305489) (width 0.25) (layer "F.Cu") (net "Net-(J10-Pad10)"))
 (segment (start 129.114511 31.305489) (end 129.114511 29.228501) (width 0.25) (layer "F.Cu") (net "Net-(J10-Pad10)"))
 (segment (start 126.574511 28.540489) (end 125.4 29.715) (width 0.25) (layer "F.Cu") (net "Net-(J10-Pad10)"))
 (via (at 126.22 34.2) (size 0.8) (drill 0.4) (layers "F.Cu" "B.Cu") (capping no) (covering (front no) (back no))
  (plugging (front no) (back no)) (filling no) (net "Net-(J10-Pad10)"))
 (segment (start 47.11 33.24601) (end 50.64101 29.715) (width 0.25) (layer "B.Cu") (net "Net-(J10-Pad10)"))
 (segment (start 47.11 33.94) (end 47.11 33.24601) (width 0.25) (layer "B.Cu") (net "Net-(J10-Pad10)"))
 (segment (start 47.76 34.59) (end 47.11 33.94) (width 0.25) (layer "B.Cu") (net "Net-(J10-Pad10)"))
 (segment (start 50.64101 29.715) (end 51.52 29.715) (width 0.25) (layer "B.Cu") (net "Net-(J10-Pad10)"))
 (segment (start 126.22 34.2) (end 125.83 34.59) (width 0.25) (layer "B.Cu") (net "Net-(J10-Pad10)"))
 (segment (start 125.83 34.59) (end 47.76 34.59) (width 0.25) (layer "B.Cu") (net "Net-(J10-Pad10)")))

